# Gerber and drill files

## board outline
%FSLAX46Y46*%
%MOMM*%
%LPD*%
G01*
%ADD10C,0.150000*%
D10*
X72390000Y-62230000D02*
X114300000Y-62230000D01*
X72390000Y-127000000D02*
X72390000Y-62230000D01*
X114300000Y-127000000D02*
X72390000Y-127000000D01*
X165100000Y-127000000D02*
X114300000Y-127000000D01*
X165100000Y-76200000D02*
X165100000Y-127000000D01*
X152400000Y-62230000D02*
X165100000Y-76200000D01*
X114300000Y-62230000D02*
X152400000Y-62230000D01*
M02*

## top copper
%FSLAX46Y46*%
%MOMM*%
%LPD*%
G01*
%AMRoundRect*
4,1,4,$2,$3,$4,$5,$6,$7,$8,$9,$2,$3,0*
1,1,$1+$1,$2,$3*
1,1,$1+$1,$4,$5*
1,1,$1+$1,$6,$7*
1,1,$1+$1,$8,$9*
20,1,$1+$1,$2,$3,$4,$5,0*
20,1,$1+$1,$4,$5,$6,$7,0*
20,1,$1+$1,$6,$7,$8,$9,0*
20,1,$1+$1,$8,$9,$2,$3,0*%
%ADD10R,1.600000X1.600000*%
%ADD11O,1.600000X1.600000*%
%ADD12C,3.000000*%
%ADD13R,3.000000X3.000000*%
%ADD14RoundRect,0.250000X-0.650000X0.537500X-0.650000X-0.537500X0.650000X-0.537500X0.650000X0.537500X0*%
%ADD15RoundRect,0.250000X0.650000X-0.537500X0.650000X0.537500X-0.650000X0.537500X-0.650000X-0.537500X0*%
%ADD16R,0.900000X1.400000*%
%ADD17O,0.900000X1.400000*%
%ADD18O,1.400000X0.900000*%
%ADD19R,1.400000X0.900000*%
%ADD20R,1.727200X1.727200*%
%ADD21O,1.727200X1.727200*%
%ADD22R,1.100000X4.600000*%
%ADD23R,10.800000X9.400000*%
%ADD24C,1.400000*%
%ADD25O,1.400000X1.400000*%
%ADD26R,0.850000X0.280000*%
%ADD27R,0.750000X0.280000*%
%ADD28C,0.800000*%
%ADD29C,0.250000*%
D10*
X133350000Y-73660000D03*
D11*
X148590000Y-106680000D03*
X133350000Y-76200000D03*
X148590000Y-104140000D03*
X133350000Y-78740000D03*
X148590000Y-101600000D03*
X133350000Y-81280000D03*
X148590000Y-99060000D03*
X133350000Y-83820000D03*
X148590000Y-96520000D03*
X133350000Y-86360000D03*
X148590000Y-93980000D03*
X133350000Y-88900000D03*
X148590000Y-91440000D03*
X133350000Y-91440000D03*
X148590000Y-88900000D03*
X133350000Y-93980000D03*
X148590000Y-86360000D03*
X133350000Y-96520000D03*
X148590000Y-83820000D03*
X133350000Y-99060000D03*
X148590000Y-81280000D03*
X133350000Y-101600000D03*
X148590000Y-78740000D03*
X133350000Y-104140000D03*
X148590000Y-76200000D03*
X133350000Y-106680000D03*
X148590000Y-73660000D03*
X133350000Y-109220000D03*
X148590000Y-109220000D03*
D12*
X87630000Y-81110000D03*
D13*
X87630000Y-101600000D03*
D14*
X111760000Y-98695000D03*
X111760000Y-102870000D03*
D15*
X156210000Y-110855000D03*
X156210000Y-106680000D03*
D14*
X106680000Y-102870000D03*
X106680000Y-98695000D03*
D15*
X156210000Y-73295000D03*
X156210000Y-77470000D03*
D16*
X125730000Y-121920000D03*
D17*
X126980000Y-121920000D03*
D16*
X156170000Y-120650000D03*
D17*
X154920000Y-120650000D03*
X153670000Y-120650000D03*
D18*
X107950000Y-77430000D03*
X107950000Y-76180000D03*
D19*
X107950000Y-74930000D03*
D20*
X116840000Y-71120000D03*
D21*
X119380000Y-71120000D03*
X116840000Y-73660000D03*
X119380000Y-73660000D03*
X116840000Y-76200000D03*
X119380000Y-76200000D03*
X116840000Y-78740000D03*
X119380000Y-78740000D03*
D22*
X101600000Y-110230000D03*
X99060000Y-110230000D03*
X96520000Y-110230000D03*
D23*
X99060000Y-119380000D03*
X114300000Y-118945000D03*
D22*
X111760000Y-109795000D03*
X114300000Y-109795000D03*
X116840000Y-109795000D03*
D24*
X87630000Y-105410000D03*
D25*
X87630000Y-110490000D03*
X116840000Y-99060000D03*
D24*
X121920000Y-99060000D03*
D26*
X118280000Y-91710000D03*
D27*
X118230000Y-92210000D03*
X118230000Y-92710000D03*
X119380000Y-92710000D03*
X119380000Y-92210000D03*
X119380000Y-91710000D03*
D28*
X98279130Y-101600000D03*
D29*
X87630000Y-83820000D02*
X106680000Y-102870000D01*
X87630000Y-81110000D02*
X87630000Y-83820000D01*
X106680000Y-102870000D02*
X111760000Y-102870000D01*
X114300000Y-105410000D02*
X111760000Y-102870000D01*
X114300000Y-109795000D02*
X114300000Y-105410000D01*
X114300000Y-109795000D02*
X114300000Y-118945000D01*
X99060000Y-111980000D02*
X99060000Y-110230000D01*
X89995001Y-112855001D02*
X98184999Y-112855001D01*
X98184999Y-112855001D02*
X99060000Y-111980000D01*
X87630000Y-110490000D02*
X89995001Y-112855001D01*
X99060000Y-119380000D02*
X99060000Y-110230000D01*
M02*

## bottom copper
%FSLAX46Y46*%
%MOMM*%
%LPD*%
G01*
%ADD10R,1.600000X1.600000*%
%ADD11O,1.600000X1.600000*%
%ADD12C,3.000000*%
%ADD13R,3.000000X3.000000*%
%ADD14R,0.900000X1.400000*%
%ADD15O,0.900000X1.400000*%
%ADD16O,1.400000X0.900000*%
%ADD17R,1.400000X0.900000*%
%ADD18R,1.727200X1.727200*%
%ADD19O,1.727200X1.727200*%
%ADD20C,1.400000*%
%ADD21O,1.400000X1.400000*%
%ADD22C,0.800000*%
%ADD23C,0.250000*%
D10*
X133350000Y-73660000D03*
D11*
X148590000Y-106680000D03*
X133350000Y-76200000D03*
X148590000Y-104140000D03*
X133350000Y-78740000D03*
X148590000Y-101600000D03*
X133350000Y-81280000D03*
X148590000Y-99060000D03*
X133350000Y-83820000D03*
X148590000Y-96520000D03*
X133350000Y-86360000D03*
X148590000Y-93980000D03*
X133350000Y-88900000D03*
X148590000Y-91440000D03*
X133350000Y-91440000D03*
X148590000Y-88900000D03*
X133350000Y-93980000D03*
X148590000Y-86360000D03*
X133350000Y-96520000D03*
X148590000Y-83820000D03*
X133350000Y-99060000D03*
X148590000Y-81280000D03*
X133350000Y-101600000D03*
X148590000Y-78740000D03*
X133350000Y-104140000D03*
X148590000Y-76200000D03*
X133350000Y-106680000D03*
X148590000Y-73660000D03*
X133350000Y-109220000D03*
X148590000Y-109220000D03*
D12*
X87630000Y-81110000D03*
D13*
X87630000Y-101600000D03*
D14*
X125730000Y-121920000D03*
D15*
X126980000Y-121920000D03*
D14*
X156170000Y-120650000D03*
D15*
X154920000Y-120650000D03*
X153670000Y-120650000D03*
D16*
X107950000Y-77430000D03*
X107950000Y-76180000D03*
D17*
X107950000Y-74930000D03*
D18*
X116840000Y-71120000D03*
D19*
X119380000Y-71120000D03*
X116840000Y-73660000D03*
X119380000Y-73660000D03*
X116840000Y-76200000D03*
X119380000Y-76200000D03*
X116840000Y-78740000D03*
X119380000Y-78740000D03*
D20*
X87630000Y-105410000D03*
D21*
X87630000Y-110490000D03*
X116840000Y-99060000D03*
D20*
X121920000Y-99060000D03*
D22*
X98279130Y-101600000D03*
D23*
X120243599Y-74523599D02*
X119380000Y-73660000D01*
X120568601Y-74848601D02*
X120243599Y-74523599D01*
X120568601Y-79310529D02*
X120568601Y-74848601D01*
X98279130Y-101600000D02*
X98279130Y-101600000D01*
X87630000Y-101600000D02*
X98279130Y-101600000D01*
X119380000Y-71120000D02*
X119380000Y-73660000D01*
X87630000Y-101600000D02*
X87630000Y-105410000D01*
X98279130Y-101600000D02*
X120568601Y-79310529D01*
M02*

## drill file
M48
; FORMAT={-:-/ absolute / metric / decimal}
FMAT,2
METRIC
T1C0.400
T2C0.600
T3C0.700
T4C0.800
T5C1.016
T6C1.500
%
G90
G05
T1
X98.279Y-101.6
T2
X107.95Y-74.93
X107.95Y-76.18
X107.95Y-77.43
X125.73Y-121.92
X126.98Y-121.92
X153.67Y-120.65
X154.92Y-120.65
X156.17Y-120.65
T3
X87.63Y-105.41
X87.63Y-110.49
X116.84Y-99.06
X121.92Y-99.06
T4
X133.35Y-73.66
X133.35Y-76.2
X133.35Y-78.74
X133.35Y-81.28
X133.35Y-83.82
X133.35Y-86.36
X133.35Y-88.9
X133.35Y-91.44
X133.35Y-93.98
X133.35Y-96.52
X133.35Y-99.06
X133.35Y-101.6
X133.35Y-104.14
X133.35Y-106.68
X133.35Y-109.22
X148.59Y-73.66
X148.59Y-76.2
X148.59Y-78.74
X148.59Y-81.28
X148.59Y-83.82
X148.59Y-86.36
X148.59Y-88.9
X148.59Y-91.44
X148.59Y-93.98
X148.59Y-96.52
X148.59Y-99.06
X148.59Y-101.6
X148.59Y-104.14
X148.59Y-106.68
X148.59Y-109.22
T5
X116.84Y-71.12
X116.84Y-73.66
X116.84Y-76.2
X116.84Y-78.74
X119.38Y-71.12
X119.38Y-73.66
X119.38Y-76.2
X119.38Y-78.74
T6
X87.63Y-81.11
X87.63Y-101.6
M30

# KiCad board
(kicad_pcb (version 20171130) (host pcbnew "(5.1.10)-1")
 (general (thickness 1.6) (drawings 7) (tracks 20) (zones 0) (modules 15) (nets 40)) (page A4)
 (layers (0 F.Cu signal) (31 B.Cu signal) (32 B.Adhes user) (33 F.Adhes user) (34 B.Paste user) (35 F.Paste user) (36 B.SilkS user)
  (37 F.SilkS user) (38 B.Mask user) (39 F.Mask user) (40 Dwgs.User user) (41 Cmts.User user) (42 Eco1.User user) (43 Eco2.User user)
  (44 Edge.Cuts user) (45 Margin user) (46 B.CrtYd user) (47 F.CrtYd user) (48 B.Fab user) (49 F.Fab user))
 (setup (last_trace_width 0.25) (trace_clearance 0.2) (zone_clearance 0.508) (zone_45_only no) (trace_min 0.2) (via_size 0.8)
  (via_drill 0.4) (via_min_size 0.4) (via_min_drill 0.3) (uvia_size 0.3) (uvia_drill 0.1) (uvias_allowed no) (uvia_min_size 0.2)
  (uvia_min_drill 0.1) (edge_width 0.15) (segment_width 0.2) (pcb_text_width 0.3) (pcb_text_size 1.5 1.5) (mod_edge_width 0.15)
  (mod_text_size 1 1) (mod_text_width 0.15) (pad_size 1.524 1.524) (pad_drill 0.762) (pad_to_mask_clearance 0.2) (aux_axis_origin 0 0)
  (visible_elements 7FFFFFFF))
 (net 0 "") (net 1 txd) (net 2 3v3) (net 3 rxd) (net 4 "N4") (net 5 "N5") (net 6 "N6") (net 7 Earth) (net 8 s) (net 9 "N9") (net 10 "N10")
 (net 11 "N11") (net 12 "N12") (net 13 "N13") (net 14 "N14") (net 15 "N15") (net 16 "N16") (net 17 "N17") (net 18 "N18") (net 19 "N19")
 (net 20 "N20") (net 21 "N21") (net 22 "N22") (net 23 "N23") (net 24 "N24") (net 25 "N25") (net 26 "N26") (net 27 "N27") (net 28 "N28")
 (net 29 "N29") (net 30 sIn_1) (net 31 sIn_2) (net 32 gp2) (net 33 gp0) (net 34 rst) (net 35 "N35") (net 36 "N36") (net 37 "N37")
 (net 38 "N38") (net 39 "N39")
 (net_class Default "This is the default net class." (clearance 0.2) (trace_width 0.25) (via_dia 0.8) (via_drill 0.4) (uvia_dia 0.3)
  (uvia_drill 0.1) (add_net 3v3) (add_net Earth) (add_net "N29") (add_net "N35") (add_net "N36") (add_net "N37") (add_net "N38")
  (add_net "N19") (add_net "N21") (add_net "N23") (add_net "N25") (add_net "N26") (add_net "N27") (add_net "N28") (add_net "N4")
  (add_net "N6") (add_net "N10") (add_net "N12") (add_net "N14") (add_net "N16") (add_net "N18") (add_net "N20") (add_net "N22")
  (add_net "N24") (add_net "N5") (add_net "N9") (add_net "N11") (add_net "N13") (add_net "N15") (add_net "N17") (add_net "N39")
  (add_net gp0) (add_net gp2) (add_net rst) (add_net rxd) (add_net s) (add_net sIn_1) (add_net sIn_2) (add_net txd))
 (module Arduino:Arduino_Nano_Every (layer F.Cu) (at 133.35 73.66)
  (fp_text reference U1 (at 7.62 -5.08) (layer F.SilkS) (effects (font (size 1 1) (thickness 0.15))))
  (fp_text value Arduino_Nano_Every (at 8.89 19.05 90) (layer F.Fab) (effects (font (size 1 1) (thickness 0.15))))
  (pad 1 thru_hole rect (at 0 0) (size 1.6 1.6) (drill 0.8) (layers *.Cu *.Mask) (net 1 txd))
  (pad 17 thru_hole oval (at 15.24 33.02) (size 1.6 1.6) (drill 0.8) (layers *.Cu *.Mask) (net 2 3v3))
  (pad 2 thru_hole oval (at 0 2.54) (size 1.6 1.6) (drill 0.8) (layers *.Cu *.Mask) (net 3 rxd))
  (pad 18 thru_hole oval (at 15.24 30.48) (size 1.6 1.6) (drill 0.8) (layers *.Cu *.Mask) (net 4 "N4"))
  (pad 3 thru_hole oval (at 0 5.08) (size 1.6 1.6) (drill 0.8) (layers *.Cu *.Mask) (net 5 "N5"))
  (pad 19 thru_hole oval (at 15.24 27.94) (size 1.6 1.6) (drill 0.8) (layers *.Cu *.Mask) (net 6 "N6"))
  (pad 4 thru_hole oval (at 0 7.62) (size 1.6 1.6) (drill 0.8) (layers *.Cu *.Mask) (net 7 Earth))
  (pad 20 thru_hole oval (at 15.24 25.4) (size 1.6 1.6) (drill 0.8) (layers *.Cu *.Mask) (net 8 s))
  (pad 5 thru_hole oval (at 0 10.16) (size 1.6 1.6) (drill 0.8) (layers *.Cu *.Mask) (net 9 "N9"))
  (pad 21 thru_hole oval (at 15.24 22.86) (size 1.6 1.6) (drill 0.8) (layers *.Cu *.Mask) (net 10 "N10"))
  (pad 6 thru_hole oval (at 0 12.7) (size 1.6 1.6) (drill 0.8) (layers *.Cu *.Mask) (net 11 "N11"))
  (pad 22 thru_hole oval (at 15.24 20.32) (size 1.6 1.6) (drill 0.8) (layers *.Cu *.Mask) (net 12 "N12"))
  (pad 7 thru_hole oval (at 0 15.24) (size 1.6 1.6) (drill 0.8) (layers *.Cu *.Mask) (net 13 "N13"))
  (pad 23 thru_hole oval (at 15.24 17.78) (size 1.6 1.6) (drill 0.8) (layers *.Cu *.Mask) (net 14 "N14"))
  (pad 8 thru_hole oval (at 0 17.78) (size 1.6 1.6) (drill 0.8) (layers *.Cu *.Mask) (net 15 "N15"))
  (pad 24 thru_hole oval (at 15.24 15.24) (size 1.6 1.6) (drill 0.8) (layers *.Cu *.Mask) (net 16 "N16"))
  (pad 9 thru_hole oval (at 0 20.32) (size 1.6 1.6) (drill 0.8) (layers *.Cu *.Mask) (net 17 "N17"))
  (pad 25 thru_hole oval (at 15.24 12.7) (size 1.6 1.6) (drill 0.8) (layers *.Cu *.Mask) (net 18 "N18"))
  (pad 10 thru_hole oval (at 0 22.86) (size 1.6 1.6) (drill 0.8) (layers *.Cu *.Mask) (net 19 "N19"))
  (pad 26 thru_hole oval (at 15.24 10.16) (size 1.6 1.6) (drill 0.8) (layers *.Cu *.Mask) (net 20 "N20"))
  (pad 11 thru_hole oval (at 0 25.4) (size 1.6 1.6) (drill 0.8) (layers *.Cu *.Mask) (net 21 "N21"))
  (pad 27 thru_hole oval (at 15.24 7.62) (size 1.6 1.6) (drill 0.8) (layers *.Cu *.Mask) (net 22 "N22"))
  (pad 12 thru_hole oval (at 0 27.94) (size 1.6 1.6) (drill 0.8) (layers *.Cu *.Mask) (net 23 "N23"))
  (pad 28 thru_hole oval (at 15.24 5.08) (size 1.6 1.6) (drill 0.8) (layers *.Cu *.Mask) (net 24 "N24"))
  (pad 13 thru_hole oval (at 0 30.48) (size 1.6 1.6) (drill 0.8) (layers *.Cu *.Mask) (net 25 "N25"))
  (pad 29 thru_hole oval (at 15.24 2.54) (size 1.6 1.6) (drill 0.8) (layers *.Cu *.Mask) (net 7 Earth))
  (pad 14 thru_hole oval (at 0 33.02) (size 1.6 1.6) (drill 0.8) (layers *.Cu *.Mask) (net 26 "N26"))
  (pad 30 thru_hole oval (at 15.24 0) (size 1.6 1.6) (drill 0.8) (layers *.Cu *.Mask) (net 2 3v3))
  (pad 15 thru_hole oval (at 0 35.56) (size 1.6 1.6) (drill 0.8) (layers *.Cu *.Mask) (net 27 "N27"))
  (pad 16 thru_hole oval (at 15.24 35.56) (size 1.6 1.6) (drill 0.8) (layers *.Cu *.Mask) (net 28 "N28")))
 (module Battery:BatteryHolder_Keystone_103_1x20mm (layer F.Cu) (at 87.63 101.6 90)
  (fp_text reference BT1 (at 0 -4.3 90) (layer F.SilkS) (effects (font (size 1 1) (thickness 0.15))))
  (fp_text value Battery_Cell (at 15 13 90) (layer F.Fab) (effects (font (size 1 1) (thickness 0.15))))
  (pad 2 thru_hole circle (at 20.49 0 90) (size 3 3) (drill 1.5) (layers *.Cu *.Mask) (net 7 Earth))
  (pad 1 thru_hole rect (at 0 0 90) (size 3 3) (drill 1.5) (layers *.Cu *.Mask) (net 2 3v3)))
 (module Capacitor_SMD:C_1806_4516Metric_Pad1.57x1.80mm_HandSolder (layer F.Cu) (at 111.76 100.7825 270)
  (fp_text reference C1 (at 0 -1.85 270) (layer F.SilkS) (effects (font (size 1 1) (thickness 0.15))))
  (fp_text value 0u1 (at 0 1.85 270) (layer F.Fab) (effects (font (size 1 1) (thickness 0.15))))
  (pad 1 smd roundrect (at -2.0875 0 270) (size 1.575 1.8) (layers F.Cu F.Paste F.Mask) (roundrect_rratio 0.15873) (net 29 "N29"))
  (pad 2 smd roundrect (at 2.0875 0 270) (size 1.575 1.8) (layers F.Cu F.Paste F.Mask) (roundrect_rratio 0.15873) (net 7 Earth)))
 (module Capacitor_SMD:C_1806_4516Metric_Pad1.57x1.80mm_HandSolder (layer F.Cu) (at 156.21 108.7675 90)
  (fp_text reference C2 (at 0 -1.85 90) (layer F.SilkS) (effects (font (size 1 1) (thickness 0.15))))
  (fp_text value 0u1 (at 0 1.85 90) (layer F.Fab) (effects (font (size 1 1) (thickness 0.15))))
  (pad 1 smd roundrect (at -2.0875 0 90) (size 1.575 1.8) (layers F.Cu F.Paste F.Mask) (roundrect_rratio 0.15873) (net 7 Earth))
  (pad 2 smd roundrect (at 2.0875 0 90) (size 1.575 1.8) (layers F.Cu F.Paste F.Mask) (roundrect_rratio 0.15873) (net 2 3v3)))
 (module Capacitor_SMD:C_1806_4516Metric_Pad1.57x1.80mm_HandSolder (layer F.Cu) (at 106.68 100.7825 270)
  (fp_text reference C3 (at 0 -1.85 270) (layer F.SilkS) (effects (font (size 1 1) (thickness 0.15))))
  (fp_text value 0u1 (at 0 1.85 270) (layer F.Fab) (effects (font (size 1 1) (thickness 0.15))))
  (pad 2 smd roundrect (at 2.0875 0 270) (size 1.575 1.8) (layers F.Cu F.Paste F.Mask) (roundrect_rratio 0.15873) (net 7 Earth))
  (pad 1 smd roundrect (at -2.0875 0 270) (size 1.575 1.8) (layers F.Cu F.Paste F.Mask) (roundrect_rratio 0.15873) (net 2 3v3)))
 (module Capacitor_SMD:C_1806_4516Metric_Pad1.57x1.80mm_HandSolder (layer F.Cu) (at 156.21 75.3825 90)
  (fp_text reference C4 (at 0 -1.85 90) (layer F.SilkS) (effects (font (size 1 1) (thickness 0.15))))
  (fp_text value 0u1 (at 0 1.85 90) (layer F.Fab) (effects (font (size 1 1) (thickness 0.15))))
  (pad 2 smd roundrect (at 2.0875 0 90) (size 1.575 1.8) (layers F.Cu F.Paste F.Mask) (roundrect_rratio 0.15873) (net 2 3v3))
  (pad 1 smd roundrect (at -2.0875 0 90) (size 1.575 1.8) (layers F.Cu F.Paste F.Mask) (roundrect_rratio 0.15873) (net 7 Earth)))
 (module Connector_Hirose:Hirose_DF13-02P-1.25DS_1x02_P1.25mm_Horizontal (layer F.Cu) (at 125.73 121.92)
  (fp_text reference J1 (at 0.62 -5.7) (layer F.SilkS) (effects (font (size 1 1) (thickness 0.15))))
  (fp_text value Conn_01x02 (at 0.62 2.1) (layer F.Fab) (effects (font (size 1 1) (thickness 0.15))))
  (pad 1 thru_hole rect (at 0 0) (size 0.9 1.4) (drill 0.6) (layers *.Cu *.Mask) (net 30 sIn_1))
  (pad 2 thru_hole oval (at 1.25 0) (size 0.9 1.4) (drill 0.6) (layers *.Cu *.Mask) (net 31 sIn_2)))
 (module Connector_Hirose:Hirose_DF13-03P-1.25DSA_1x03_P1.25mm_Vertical (layer F.Cu) (at 156.17 120.65 180)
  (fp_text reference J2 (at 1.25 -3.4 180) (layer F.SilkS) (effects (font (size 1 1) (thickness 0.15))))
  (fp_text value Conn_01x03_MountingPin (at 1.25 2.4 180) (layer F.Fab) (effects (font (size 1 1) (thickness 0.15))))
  (pad 1 thru_hole rect (at 0 0 180) (size 0.9 1.4) (drill 0.6) (layers *.Cu *.Mask) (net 8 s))
  (pad 2 thru_hole oval (at 1.25 0 180) (size 0.9 1.4) (drill 0.6) (layers *.Cu *.Mask) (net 2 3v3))
  (pad 3 thru_hole oval (at 2.5 0 180) (size 0.9 1.4) (drill 0.6) (layers *.Cu *.Mask) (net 7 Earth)))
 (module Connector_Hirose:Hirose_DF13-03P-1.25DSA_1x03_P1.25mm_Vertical (layer F.Cu) (at 107.95 74.93 270)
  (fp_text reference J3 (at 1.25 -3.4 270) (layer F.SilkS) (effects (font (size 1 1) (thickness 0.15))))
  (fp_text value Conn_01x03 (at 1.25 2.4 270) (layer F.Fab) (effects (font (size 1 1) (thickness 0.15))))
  (pad 3 thru_hole oval (at 2.5 0 270) (size 0.9 1.4) (drill 0.6) (layers *.Cu *.Mask) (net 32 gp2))
  (pad 2 thru_hole oval (at 1.25 0 270) (size 0.9 1.4) (drill 0.6) (layers *.Cu *.Mask) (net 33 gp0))
  (pad 1 thru_hole rect (at 0 0 270) (size 0.9 1.4) (drill 0.6) (layers *.Cu *.Mask) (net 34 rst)))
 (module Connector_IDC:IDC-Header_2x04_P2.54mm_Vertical (layer F.Cu) (at 116.84 71.12)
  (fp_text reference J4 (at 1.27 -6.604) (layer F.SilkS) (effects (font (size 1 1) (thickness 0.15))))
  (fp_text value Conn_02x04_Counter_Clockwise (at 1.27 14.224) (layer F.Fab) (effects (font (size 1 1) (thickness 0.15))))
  (pad 1 thru_hole rect (at 0 0) (size 1.7272 1.7272) (drill 1.016) (layers *.Cu *.Mask) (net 1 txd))
  (pad 2 thru_hole oval (at 2.54 0) (size 1.7272 1.7272) (drill 1.016) (layers *.Cu *.Mask) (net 2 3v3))
  (pad 3 thru_hole oval (at 0 2.54) (size 1.7272 1.7272) (drill 1.016) (layers *.Cu *.Mask) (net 34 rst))
  (pad 4 thru_hole oval (at 2.54 2.54) (size 1.7272 1.7272) (drill 1.016) (layers *.Cu *.Mask) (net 2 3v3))
  (pad 5 thru_hole oval (at 0 5.08) (size 1.7272 1.7272) (drill 1.016) (layers *.Cu *.Mask) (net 3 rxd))
  (pad 6 thru_hole oval (at 2.54 5.08) (size 1.7272 1.7272) (drill 1.016) (layers *.Cu *.Mask) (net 33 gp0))
  (pad 7 thru_hole oval (at 0 7.62) (size 1.7272 1.7272) (drill 1.016) (layers *.Cu *.Mask) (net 32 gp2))
  (pad 8 thru_hole oval (at 2.54 7.62) (size 1.7272 1.7272) (drill 1.016) (layers *.Cu *.Mask) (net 7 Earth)))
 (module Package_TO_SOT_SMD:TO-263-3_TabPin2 (layer F.Cu) (at 99.06 116.005 270)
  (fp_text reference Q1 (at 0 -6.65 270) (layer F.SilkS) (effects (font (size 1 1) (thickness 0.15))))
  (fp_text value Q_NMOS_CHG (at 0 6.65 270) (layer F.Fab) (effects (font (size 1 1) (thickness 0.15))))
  (pad 1 smd rect (at -5.775 -2.54 270) (size 4.6 1.1) (layers F.Cu F.Paste F.Mask) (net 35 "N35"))
  (pad 2 smd rect (at -5.775 0 270) (size 4.6 1.1) (layers F.Cu F.Paste F.Mask) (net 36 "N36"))
  (pad 3 smd rect (at -5.775 2.54 270) (size 4.6 1.1) (layers F.Cu F.Paste F.Mask) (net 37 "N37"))
  (pad 2 smd rect (at 3.375 0 270) (size 9.4 10.8) (layers F.Cu F.Mask) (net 36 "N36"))
  (pad "" smd rect (at 5.8 2.775 270) (size 4.55 5.25) (layers F.Paste))
  (pad "" smd rect (at 0.95 -2.775 270) (size 4.55 5.25) (layers F.Paste))
  (pad "" smd rect (at 5.8 -2.775 270) (size 4.55 5.25) (layers F.Paste))
  (pad "" smd rect (at 0.95 2.775 270) (size 4.55 5.25) (layers F.Paste)))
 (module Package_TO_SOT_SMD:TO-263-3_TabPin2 (layer F.Cu) (at 114.3 115.57 270)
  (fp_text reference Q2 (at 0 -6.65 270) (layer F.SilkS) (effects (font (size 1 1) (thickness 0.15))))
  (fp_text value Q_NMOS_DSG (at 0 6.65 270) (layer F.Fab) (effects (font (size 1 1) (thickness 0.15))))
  (pad "" smd rect (at 0.95 2.775 270) (size 4.55 5.25) (layers F.Paste))
  (pad "" smd rect (at 5.8 -2.775 270) (size 4.55 5.25) (layers F.Paste))
  (pad "" smd rect (at 0.95 -2.775 270) (size 4.55 5.25) (layers F.Paste))
  (pad "" smd rect (at 5.8 2.775 270) (size 4.55 5.25) (layers F.Paste))
  (pad 2 smd rect (at 3.375 0 270) (size 9.4 10.8) (layers F.Cu F.Mask) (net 7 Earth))
  (pad 3 smd rect (at -5.775 2.54 270) (size 4.6 1.1) (layers F.Cu F.Paste F.Mask) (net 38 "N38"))
  (pad 2 smd rect (at -5.775 0 270) (size 4.6 1.1) (layers F.Cu F.Paste F.Mask) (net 7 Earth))
  (pad 1 smd rect (at -5.775 -2.54 270) (size 4.6 1.1) (layers F.Cu F.Paste F.Mask) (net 35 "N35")))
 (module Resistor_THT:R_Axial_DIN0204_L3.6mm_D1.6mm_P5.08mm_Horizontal (layer F.Cu) (at 87.63 105.41 270)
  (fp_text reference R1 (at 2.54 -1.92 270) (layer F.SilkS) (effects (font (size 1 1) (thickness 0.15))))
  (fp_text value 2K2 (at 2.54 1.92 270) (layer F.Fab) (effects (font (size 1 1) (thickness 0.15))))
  (pad 1 thru_hole circle (at 0 0 270) (size 1.4 1.4) (drill 0.7) (layers *.Cu *.Mask) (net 2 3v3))
  (pad 2 thru_hole oval (at 5.08 0 270) (size 1.4 1.4) (drill 0.7) (layers *.Cu *.Mask) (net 36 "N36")))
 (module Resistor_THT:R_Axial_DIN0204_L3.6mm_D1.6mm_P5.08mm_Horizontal (layer F.Cu) (at 121.92 99.06 180)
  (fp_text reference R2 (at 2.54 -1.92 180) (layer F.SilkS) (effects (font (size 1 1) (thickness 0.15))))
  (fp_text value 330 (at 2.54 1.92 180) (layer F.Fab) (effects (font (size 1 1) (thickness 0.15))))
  (pad 2 thru_hole oval (at 5.08 0 180) (size 1.4 1.4) (drill 0.7) (layers *.Cu *.Mask) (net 29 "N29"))
  (pad 1 thru_hole circle (at 0 0 180) (size 1.4 1.4) (drill 0.7) (layers *.Cu *.Mask) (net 2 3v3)))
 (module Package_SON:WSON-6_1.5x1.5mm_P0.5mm (layer F.Cu) (at 118.805 92.21)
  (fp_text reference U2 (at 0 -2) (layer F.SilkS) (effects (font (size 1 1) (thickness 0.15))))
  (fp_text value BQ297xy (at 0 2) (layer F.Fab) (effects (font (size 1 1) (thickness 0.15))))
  (pad 1 smd rect (at -0.525 -0.5 270) (size 0.28 0.85) (layers F.Cu F.Paste F.Mask) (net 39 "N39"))
  (pad 2 smd rect (at -0.575 0 270) (size 0.28 0.75) (layers F.Cu F.Paste F.Mask) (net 37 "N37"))
  (pad 3 smd rect (at -0.575 0.5 270) (size 0.28 0.75) (layers F.Cu F.Paste F.Mask) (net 38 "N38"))
  (pad 4 smd rect (at 0.575 0.5 270) (size 0.28 0.75) (layers F.Cu F.Paste F.Mask) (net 7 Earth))
  (pad 5 smd rect (at 0.575 0 270) (size 0.28 0.75) (layers F.Cu F.Paste F.Mask) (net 29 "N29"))
  (pad 6 smd rect (at 0.575 -0.5 270) (size 0.28 0.75) (layers F.Cu F.Paste F.Mask) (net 2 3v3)))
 (gr_line (start 72.39 62.23) (end 114.3 62.23) (layer Edge.Cuts) (width 0.15))
 (gr_line (start 72.39 127) (end 72.39 62.23) (layer Edge.Cuts) (width 0.15))
 (gr_line (start 114.3 127) (end 72.39 127) (layer Edge.Cuts) (width 0.15))
 (gr_line (start 165.1 127) (end 114.3 127) (layer Edge.Cuts) (width 0.15))
 (gr_line (start 165.1 76.2) (end 165.1 127) (layer Edge.Cuts) (width 0.15))
 (gr_line (start 152.4 62.23) (end 165.1 76.2) (layer Edge.Cuts) (width 0.15))
 (gr_line (start 114.3 62.23) (end 152.4 62.23) (layer Edge.Cuts) (width 0.15))
 (segment (start 87.63 83.82) (end 106.68 102.87) (width 0.25) (layer F.Cu) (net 7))
 (segment (start 87.63 81.11) (end 87.63 83.82) (width 0.25) (layer F.Cu) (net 7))
 (segment (start 106.68 102.87) (end 111.76 102.87) (width 0.25) (layer F.Cu) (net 7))
 (segment (start 114.3 105.41) (end 111.76 102.87) (width 0.25) (layer F.Cu) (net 7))
 (segment (start 114.3 109.795) (end 114.3 105.41) (width 0.25) (layer F.Cu) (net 7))
 (segment (start 114.3 109.795) (end 114.3 118.945) (width 0.25) (layer F.Cu) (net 7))
 (segment (start 120.243599 74.523599) (end 119.38 73.66) (width 0.25) (layer B.Cu) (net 2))
 (segment (start 120.568601 74.848601) (end 120.243599 74.523599) (width 0.25) (layer B.Cu) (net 2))
 (segment (start 120.568601 79.310529) (end 120.568601 74.848601) (width 0.25) (layer B.Cu) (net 2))
 (segment (start 98.27913 101.6) (end 98.27913 101.6) (width 0.25) (layer B.Cu) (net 2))
 (segment (start 87.63 101.6) (end 98.27913 101.6) (width 0.25) (layer B.Cu) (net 2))
 (segment (start 119.38 71.12) (end 119.38 73.66) (width 0.25) (layer B.Cu) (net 2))
 (segment (start 87.63 101.6) (end 87.63 105.41) (width 0.25) (layer B.Cu) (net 2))
 (segment (start 98.27913 101.6) (end 120.568601 79.310529) (width 0.25) (layer B.Cu) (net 2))
 (via (at 98.27913 101.6) (size 0.8) (drill 0.4) (layers F.Cu B.Cu) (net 2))
 (segment (start 99.06 111.98) (end 99.06 110.23) (width 0.25) (layer F.Cu) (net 36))
 (segment (start 89.995001 112.855001) (end 98.184999 112.855001) (width 0.25) (layer F.Cu) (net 36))
 (segment (start 98.184999 112.855001) (end 99.06 111.98) (width 0.25) (layer F.Cu) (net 36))
 (segment (start 87.63 110.49) (end 89.995001 112.855001) (width 0.25) (layer F.Cu) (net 36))
 (segment (start 99.06 119.38) (end 99.06 110.23) (width 0.25) (layer F.Cu) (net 36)))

